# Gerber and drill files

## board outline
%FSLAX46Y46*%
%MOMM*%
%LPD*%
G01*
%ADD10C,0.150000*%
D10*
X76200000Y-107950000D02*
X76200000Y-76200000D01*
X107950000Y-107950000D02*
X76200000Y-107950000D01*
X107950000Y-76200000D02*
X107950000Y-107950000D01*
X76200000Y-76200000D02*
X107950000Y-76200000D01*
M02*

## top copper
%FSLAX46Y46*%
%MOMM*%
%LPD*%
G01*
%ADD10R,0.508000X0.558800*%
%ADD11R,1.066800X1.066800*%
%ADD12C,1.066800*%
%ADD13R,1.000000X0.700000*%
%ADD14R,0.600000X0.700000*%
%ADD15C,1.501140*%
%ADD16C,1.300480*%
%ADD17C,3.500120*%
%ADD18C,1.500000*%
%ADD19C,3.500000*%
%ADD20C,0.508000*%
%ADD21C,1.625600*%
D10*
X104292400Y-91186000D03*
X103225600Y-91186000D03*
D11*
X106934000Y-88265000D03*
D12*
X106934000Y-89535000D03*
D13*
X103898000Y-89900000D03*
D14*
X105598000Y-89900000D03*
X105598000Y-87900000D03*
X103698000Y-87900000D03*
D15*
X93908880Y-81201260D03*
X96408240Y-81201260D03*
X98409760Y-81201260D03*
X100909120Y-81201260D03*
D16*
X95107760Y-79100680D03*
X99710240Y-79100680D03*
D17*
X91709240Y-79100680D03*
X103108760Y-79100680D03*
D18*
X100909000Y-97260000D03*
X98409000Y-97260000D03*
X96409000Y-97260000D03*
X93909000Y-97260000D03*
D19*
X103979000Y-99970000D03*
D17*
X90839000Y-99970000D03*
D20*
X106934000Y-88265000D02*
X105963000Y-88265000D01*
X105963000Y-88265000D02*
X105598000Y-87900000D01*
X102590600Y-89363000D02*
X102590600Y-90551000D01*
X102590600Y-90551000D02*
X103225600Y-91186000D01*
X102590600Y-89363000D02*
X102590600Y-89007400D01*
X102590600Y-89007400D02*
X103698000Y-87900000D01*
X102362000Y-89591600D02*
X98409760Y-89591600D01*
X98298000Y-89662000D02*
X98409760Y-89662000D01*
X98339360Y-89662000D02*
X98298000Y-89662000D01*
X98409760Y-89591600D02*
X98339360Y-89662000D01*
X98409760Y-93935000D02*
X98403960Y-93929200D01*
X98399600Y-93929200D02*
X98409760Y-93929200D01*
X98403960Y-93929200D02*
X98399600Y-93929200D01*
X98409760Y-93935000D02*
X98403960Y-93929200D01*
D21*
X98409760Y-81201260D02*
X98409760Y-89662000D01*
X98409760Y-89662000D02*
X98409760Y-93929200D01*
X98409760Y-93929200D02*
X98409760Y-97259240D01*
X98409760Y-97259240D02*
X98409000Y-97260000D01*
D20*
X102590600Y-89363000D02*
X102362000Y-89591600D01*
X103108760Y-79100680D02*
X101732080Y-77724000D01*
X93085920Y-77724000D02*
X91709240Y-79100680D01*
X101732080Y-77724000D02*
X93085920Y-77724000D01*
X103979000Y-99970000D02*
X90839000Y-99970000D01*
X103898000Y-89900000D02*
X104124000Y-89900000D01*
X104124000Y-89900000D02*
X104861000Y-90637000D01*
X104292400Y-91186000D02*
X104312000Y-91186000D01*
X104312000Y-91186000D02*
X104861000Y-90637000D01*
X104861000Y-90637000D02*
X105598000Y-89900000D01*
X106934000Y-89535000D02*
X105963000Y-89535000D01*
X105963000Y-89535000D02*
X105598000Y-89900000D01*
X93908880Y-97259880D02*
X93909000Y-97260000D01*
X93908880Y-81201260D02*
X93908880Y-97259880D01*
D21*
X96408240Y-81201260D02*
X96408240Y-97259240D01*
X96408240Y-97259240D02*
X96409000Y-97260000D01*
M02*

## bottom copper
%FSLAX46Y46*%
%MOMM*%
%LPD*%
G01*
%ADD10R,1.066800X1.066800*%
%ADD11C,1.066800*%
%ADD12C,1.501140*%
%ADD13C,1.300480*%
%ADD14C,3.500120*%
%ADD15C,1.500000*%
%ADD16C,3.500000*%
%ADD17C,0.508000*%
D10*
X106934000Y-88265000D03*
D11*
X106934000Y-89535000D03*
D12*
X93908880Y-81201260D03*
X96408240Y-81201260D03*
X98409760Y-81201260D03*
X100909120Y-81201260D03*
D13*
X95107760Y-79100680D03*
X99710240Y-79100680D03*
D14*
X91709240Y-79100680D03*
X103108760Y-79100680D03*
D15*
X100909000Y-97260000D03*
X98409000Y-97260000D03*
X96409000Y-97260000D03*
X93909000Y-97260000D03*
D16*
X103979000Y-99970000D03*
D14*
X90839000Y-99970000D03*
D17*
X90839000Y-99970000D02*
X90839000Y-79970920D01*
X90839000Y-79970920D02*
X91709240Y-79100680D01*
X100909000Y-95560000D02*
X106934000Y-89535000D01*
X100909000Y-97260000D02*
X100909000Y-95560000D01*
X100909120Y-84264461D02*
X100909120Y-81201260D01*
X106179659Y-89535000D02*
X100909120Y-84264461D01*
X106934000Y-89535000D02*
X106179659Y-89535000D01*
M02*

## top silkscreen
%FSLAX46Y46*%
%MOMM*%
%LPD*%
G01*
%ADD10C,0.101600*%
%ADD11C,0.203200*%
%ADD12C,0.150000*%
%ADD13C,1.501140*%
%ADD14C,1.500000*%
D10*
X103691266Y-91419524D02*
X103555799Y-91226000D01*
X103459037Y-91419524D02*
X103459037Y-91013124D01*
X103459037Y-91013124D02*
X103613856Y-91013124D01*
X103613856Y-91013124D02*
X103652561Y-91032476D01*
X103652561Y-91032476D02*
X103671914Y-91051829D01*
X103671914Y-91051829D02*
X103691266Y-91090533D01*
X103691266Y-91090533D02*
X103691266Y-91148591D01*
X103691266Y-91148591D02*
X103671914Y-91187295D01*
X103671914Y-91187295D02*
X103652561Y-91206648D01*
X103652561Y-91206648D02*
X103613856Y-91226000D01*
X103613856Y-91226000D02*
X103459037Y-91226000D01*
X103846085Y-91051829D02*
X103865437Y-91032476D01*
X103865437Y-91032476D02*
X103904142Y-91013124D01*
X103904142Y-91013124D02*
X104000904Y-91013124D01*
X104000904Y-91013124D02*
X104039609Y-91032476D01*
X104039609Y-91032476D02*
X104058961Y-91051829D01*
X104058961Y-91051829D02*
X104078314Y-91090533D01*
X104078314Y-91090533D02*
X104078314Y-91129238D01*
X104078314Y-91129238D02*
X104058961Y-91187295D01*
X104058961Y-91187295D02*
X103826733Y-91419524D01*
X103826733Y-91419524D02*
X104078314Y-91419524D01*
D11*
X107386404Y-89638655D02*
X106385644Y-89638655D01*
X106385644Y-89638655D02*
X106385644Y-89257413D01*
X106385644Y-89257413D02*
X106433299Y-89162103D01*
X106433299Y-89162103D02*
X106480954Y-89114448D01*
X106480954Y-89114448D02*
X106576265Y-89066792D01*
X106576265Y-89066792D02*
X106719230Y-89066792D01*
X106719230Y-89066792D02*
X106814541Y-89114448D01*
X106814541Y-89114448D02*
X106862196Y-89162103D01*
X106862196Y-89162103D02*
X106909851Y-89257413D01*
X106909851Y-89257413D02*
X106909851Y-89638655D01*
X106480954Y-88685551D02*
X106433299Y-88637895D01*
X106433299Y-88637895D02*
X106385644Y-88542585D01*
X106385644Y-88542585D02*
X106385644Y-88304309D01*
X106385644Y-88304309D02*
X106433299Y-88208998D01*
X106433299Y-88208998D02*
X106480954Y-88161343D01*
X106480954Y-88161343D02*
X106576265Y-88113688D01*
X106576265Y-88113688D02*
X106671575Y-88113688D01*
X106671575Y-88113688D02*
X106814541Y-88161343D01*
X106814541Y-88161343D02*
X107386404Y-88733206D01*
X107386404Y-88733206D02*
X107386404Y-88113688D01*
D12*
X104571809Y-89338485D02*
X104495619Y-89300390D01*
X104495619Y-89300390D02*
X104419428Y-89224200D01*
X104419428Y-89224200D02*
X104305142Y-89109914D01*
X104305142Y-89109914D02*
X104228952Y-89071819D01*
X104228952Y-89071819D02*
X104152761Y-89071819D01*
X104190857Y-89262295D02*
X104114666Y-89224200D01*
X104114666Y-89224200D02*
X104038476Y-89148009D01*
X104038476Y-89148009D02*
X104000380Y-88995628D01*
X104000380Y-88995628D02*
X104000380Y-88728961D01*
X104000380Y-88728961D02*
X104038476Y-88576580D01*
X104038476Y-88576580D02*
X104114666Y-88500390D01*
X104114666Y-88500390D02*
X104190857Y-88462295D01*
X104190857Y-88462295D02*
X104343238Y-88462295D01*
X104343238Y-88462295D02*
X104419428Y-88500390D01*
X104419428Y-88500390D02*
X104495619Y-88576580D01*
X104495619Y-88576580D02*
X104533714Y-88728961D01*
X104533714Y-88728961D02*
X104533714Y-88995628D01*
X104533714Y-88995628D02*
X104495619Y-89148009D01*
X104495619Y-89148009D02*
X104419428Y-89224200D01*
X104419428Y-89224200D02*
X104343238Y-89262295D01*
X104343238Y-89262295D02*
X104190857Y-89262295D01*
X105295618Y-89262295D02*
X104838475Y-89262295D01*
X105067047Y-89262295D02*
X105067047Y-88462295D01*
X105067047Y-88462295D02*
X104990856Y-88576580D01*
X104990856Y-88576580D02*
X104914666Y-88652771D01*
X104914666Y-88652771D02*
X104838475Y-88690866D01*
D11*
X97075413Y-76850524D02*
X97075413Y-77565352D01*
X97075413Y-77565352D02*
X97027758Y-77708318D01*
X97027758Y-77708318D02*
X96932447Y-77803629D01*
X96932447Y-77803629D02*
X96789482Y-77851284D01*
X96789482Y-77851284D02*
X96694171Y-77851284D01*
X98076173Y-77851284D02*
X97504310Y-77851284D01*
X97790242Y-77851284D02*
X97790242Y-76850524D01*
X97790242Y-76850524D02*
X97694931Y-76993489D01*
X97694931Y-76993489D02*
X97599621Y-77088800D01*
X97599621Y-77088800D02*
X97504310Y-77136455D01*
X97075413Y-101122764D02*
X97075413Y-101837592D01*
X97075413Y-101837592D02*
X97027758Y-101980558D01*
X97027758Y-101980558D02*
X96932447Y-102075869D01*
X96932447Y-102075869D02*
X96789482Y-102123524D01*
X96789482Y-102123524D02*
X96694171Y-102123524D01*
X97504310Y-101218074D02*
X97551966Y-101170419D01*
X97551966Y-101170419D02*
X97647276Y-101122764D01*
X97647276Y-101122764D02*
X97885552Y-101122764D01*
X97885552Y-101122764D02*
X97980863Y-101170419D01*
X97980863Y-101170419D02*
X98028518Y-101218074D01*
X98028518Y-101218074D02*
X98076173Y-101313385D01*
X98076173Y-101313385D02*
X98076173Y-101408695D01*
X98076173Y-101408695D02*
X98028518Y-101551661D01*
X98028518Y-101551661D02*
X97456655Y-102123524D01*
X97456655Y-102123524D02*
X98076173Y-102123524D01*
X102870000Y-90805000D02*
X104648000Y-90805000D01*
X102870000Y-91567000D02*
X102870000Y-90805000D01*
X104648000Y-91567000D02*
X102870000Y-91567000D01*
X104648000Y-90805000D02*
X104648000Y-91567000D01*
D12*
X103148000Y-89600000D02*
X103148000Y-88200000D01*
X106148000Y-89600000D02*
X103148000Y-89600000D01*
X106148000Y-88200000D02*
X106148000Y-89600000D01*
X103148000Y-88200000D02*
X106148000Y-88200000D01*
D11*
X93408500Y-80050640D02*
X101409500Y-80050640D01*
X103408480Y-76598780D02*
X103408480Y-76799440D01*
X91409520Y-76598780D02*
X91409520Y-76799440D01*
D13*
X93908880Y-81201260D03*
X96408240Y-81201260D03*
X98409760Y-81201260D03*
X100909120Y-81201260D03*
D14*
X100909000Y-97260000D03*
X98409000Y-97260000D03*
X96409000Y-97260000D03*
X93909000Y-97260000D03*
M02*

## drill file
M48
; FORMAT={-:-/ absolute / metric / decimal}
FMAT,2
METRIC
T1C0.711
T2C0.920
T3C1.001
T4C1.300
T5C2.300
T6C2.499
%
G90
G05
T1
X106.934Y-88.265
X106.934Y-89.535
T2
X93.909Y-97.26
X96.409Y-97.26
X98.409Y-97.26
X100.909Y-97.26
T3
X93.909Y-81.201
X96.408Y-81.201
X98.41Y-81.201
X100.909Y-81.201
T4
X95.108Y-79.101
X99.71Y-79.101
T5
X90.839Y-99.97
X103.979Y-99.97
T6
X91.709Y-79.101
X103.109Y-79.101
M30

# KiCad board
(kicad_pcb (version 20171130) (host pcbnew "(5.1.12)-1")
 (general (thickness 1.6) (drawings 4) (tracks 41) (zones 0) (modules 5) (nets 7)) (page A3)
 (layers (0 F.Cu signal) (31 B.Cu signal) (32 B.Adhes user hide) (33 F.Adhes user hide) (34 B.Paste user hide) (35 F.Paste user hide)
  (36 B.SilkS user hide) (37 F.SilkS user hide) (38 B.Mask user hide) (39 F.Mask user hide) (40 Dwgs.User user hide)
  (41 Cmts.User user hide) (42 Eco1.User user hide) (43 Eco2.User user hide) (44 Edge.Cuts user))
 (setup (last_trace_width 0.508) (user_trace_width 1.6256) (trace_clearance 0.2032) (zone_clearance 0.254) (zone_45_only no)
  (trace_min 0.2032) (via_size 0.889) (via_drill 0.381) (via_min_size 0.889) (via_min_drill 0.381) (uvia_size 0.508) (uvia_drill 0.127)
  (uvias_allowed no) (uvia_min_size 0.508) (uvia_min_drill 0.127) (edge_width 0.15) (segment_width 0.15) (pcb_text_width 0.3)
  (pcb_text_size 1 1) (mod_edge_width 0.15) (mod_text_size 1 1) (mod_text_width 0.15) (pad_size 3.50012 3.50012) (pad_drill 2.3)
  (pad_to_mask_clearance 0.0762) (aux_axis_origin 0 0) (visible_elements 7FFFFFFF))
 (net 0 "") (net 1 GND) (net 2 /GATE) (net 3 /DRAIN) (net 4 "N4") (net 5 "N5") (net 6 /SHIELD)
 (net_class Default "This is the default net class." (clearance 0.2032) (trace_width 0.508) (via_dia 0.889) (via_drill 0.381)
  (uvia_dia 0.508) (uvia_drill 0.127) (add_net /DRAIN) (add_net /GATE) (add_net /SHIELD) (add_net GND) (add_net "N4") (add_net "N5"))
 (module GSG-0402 (layer F.Cu) (at 103.759 91.186) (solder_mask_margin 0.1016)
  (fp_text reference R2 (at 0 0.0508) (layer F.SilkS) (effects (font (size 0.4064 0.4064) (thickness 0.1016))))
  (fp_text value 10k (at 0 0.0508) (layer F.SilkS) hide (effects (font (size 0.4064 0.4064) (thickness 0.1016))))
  (fp_line (start -0.889 -0.381) (end 0.889 -0.381) (layer F.SilkS) (width 0.2032))
  (fp_line (start -0.889 0.381) (end -0.889 -0.381) (layer F.SilkS) (width 0.2032))
  (fp_line (start 0.889 0.381) (end -0.889 0.381) (layer F.SilkS) (width 0.2032))
  (fp_line (start 0.889 -0.381) (end 0.889 0.381) (layer F.SilkS) (width 0.2032))
  (pad 2 smd rect (at 0.5334 0) (size 0.508 0.5588) (layers F.Cu F.Paste F.Mask) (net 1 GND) (solder_mask_margin 0.1016))
  (pad 1 smd rect (at -0.5334 0) (size 0.508 0.5588) (layers F.Cu F.Paste F.Mask) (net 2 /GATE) (die_length -1518.485687)
   (solder_mask_margin 0.1016)))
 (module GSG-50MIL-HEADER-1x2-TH (layer F.Cu) (at 106.934 88.9 270)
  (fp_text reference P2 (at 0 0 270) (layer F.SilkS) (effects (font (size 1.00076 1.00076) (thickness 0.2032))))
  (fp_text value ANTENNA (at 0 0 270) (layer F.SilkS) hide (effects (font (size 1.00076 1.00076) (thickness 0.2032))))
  (pad 1 thru_hole rect (at -0.635 0 270) (size 1.0668 1.0668) (drill 0.7112) (layers *.Cu *.Mask) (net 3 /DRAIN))
  (pad 2 thru_hole circle (at 0.635 0 270) (size 1.0668 1.0668) (drill 0.7112) (layers *.Cu *.Mask) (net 1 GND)))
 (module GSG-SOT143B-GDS (layer F.Cu) (at 104.648 88.9)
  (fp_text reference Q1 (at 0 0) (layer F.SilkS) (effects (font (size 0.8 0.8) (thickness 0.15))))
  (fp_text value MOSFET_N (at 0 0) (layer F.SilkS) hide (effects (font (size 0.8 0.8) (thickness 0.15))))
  (fp_line (start -1.5 0.7) (end -1.5 -0.7) (layer F.SilkS) (width 0.15))
  (fp_line (start 1.5 0.7) (end -1.5 0.7) (layer F.SilkS) (width 0.15))
  (fp_line (start 1.5 -0.7) (end 1.5 0.7) (layer F.SilkS) (width 0.15))
  (fp_line (start -1.5 -0.7) (end 1.5 -0.7) (layer F.SilkS) (width 0.15))
  (pad B smd rect (at -0.75 1) (size 1 0.7) (layers F.Cu F.Paste F.Mask) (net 1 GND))
  (pad S smd rect (at 0.95 1) (size 0.6 0.7) (layers F.Cu F.Paste F.Mask) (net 1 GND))
  (pad D smd rect (at 0.95 -1) (size 0.6 0.7) (layers F.Cu F.Paste F.Mask) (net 3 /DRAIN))
  (pad G smd rect (at -0.95 -1) (size 0.6 0.7) (layers F.Cu F.Paste F.Mask) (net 2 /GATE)))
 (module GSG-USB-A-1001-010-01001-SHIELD (layer F.Cu) (at 97.409 76.2 180)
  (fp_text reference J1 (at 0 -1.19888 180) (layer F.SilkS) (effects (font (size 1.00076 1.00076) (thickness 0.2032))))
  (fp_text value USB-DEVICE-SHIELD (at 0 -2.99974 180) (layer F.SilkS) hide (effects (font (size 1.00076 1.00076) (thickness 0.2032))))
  (fp_line (start 4.0005 -3.85064) (end -4.0005 -3.85064) (layer F.SilkS) (width 0.2032))
  (fp_line (start -5.99948 -0.39878) (end -5.99948 -0.59944) (layer F.SilkS) (width 0.2032))
  (fp_line (start 5.99948 -0.39878) (end 5.99948 -0.59944) (layer F.SilkS) (width 0.2032))
  (pad 1 thru_hole circle (at 3.50012 -5.00126 180) (size 1.50114 1.50114) (drill 1.00076) (layers *.Cu *.Mask F.SilkS) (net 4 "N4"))
  (pad 2 thru_hole circle (at 1.00076 -5.00126 180) (size 1.50114 1.50114) (drill 1.00076) (layers *.Cu *.Mask F.SilkS) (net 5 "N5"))
  (pad 3 thru_hole circle (at -1.00076 -5.00126 180) (size 1.50114 1.50114) (drill 1.00076) (layers *.Cu *.Mask F.SilkS) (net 2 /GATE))
  (pad 4 thru_hole circle (at -3.50012 -5.00126 180) (size 1.50114 1.50114) (drill 1.00076) (layers *.Cu *.Mask F.SilkS) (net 1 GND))
  (pad "" thru_hole circle (at 2.30124 -2.90068 180) (size 1.30048 1.30048) (drill 1.30048) (layers *.Cu *.Mask) (clearance -0.09906))
  (pad "" thru_hole circle (at -2.30124 -2.90068 180) (size 1.30048 1.30048) (drill 1.30048) (layers *.Cu *.Mask) (clearance -0.09906))
  (pad 5 thru_hole circle (at 5.69976 -2.90068 180) (size 3.50012 3.50012) (drill 2.49936) (layers *.Cu *.Mask) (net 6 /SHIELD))
  (pad 5 thru_hole circle (at -5.69976 -2.90068 180) (size 3.50012 3.50012) (drill 2.49936) (layers *.Cu *.Mask) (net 6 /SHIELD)))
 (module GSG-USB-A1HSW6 (layer F.Cu) (at 97.409 102.87)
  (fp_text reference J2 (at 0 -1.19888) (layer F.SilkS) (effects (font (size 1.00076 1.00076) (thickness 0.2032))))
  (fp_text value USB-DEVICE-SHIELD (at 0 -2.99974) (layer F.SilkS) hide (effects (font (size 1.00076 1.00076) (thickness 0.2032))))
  (pad 4 thru_hole circle (at 3.5 -5.61) (size 1.5 1.5) (drill 0.92) (layers *.Cu *.Mask F.SilkS) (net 1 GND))
  (pad 3 thru_hole circle (at 1 -5.61) (size 1.5 1.5) (drill 0.92) (layers *.Cu *.Mask F.SilkS) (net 2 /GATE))
  (pad 2 thru_hole circle (at -1 -5.61) (size 1.5 1.5) (drill 0.92) (layers *.Cu *.Mask F.SilkS) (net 5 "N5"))
  (pad 1 thru_hole circle (at -3.5 -5.61) (size 1.5 1.5) (drill 0.92) (layers *.Cu *.Mask F.SilkS) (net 4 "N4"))
  (pad 5 thru_hole circle (at 6.57 -2.9) (size 3.5 3.5) (drill 2.3) (layers *.Cu *.Mask) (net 6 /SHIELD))
  (pad 5 thru_hole circle (at -6.57 -2.9) (size 3.50012 3.50012) (drill 2.3) (layers *.Cu *.Mask) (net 6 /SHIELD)))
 (gr_line (start 76.2 107.95) (end 76.2 76.2) (angle 90) (layer Edge.Cuts) (width 0.15))
 (gr_line (start 107.95 107.95) (end 76.2 107.95) (angle 90) (layer Edge.Cuts) (width 0.15))
 (gr_line (start 107.95 76.2) (end 107.95 107.95) (angle 90) (layer Edge.Cuts) (width 0.15))
 (gr_line (start 76.2 76.2) (end 107.95 76.2) (angle 90) (layer Edge.Cuts) (width 0.15))
 (segment (start 106.934 88.265) (end 105.963 88.265) (width 0.508) (layer F.Cu) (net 3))
 (segment (start 105.963 88.265) (end 105.598 87.9) (width 0.508) (layer F.Cu) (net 3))
 (segment (start 102.5906 89.363) (end 102.5906 90.551) (width 0.508) (layer F.Cu) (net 2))
 (segment (start 102.5906 90.551) (end 103.2256 91.186) (width 0.508) (layer F.Cu) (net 2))
 (segment (start 102.5906 89.363) (end 102.5906 89.0074) (width 0.508) (layer F.Cu) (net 2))
 (segment (start 102.5906 89.0074) (end 103.698 87.9) (width 0.508) (layer F.Cu) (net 2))
 (segment (start 102.362 89.5916) (end 98.40976 89.5916) (width 0.508) (layer F.Cu) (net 2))
 (segment (start 98.298 89.662) (end 98.40976 89.662) (width 0.508) (layer F.Cu) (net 2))
 (segment (start 98.33936 89.662) (end 98.298 89.662) (width 0.508) (layer F.Cu) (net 2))
 (segment (start 98.40976 89.5916) (end 98.33936 89.662) (width 0.508) (layer F.Cu) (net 2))
 (segment (start 98.40976 93.935) (end 98.40396 93.9292) (width 0.508) (layer F.Cu) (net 2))
 (segment (start 98.3996 93.9292) (end 98.40976 93.9292) (width 0.508) (layer F.Cu) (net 2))
 (segment (start 98.40396 93.9292) (end 98.3996 93.9292) (width 0.508) (layer F.Cu) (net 2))
 (segment (start 98.40976 93.935) (end 98.40396 93.9292) (width 0.508) (layer F.Cu) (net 2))
 (segment (start 98.40976 81.20126) (end 98.40976 89.662) (width 1.6256) (layer F.Cu) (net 2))
 (segment (start 98.40976 89.662) (end 98.40976 93.9292) (width 1.6256) (layer F.Cu) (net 2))
 (segment (start 98.40976 93.9292) (end 98.40976 97.25924) (width 1.6256) (layer F.Cu) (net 2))
 (segment (start 98.40976 97.25924) (end 98.409 97.26) (width 1.6256) (layer F.Cu) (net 2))
 (segment (start 102.5906 89.363) (end 102.362 89.5916) (width 0.508) (layer F.Cu) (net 2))
 (segment (start 103.10876 79.10068) (end 101.73208 77.724) (width 0.508) (layer F.Cu) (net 6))
 (segment (start 93.08592 77.724) (end 91.70924 79.10068) (width 0.508) (layer F.Cu) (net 6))
 (segment (start 101.73208 77.724) (end 93.08592 77.724) (width 0.508) (layer F.Cu) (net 6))
 (segment (start 103.979 99.97) (end 90.839 99.97) (width 0.508) (layer F.Cu) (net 6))
 (segment (start 90.839 99.97) (end 90.839 79.97092) (width 0.508) (layer B.Cu) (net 6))
 (segment (start 90.839 79.97092) (end 91.70924 79.10068) (width 0.508) (layer B.Cu) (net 6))
 (segment (start 103.898 89.9) (end 104.124 89.9) (width 0.508) (layer F.Cu) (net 1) (status C00000))
 (segment (start 104.124 89.9) (end 104.861 90.637) (width 0.508) (layer F.Cu) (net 1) (status 400000))
 (segment (start 104.2924 91.186) (end 104.312 91.186) (width 0.508) (layer F.Cu) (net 1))
 (segment (start 104.312 91.186) (end 104.861 90.637) (width 0.508) (layer F.Cu) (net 1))
 (segment (start 104.861 90.637) (end 105.598 89.9) (width 0.508) (layer F.Cu) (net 1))
 (segment (start 106.934 89.535) (end 105.963 89.535) (width 0.508) (layer F.Cu) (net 1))
 (segment (start 105.963 89.535) (end 105.598 89.9) (width 0.508) (layer F.Cu) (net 1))
 (segment (start 100.909 95.56) (end 106.934 89.535) (width 0.508) (layer B.Cu) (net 1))
 (segment (start 100.909 97.26) (end 100.909 95.56) (width 0.508) (layer B.Cu) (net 1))
 (segment (start 100.90912 84.264461) (end 100.90912 81.20126) (width 0.508) (layer B.Cu) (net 1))
 (segment (start 106.179659 89.535) (end 100.90912 84.264461) (width 0.508) (layer B.Cu) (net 1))
 (segment (start 106.934 89.535) (end 106.179659 89.535) (width 0.508) (layer B.Cu) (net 1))
 (segment (start 93.90888 97.25988) (end 93.909 97.26) (width 0.508) (layer F.Cu) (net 4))
 (segment (start 93.90888 81.20126) (end 93.90888 97.25988) (width 0.508) (layer F.Cu) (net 4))
 (segment (start 96.40824 81.20126) (end 96.40824 97.25924) (width 1.6256) (layer F.Cu) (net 5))
 (segment (start 96.40824 97.25924) (end 96.409 97.26) (width 1.6256) (layer F.Cu) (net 5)))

